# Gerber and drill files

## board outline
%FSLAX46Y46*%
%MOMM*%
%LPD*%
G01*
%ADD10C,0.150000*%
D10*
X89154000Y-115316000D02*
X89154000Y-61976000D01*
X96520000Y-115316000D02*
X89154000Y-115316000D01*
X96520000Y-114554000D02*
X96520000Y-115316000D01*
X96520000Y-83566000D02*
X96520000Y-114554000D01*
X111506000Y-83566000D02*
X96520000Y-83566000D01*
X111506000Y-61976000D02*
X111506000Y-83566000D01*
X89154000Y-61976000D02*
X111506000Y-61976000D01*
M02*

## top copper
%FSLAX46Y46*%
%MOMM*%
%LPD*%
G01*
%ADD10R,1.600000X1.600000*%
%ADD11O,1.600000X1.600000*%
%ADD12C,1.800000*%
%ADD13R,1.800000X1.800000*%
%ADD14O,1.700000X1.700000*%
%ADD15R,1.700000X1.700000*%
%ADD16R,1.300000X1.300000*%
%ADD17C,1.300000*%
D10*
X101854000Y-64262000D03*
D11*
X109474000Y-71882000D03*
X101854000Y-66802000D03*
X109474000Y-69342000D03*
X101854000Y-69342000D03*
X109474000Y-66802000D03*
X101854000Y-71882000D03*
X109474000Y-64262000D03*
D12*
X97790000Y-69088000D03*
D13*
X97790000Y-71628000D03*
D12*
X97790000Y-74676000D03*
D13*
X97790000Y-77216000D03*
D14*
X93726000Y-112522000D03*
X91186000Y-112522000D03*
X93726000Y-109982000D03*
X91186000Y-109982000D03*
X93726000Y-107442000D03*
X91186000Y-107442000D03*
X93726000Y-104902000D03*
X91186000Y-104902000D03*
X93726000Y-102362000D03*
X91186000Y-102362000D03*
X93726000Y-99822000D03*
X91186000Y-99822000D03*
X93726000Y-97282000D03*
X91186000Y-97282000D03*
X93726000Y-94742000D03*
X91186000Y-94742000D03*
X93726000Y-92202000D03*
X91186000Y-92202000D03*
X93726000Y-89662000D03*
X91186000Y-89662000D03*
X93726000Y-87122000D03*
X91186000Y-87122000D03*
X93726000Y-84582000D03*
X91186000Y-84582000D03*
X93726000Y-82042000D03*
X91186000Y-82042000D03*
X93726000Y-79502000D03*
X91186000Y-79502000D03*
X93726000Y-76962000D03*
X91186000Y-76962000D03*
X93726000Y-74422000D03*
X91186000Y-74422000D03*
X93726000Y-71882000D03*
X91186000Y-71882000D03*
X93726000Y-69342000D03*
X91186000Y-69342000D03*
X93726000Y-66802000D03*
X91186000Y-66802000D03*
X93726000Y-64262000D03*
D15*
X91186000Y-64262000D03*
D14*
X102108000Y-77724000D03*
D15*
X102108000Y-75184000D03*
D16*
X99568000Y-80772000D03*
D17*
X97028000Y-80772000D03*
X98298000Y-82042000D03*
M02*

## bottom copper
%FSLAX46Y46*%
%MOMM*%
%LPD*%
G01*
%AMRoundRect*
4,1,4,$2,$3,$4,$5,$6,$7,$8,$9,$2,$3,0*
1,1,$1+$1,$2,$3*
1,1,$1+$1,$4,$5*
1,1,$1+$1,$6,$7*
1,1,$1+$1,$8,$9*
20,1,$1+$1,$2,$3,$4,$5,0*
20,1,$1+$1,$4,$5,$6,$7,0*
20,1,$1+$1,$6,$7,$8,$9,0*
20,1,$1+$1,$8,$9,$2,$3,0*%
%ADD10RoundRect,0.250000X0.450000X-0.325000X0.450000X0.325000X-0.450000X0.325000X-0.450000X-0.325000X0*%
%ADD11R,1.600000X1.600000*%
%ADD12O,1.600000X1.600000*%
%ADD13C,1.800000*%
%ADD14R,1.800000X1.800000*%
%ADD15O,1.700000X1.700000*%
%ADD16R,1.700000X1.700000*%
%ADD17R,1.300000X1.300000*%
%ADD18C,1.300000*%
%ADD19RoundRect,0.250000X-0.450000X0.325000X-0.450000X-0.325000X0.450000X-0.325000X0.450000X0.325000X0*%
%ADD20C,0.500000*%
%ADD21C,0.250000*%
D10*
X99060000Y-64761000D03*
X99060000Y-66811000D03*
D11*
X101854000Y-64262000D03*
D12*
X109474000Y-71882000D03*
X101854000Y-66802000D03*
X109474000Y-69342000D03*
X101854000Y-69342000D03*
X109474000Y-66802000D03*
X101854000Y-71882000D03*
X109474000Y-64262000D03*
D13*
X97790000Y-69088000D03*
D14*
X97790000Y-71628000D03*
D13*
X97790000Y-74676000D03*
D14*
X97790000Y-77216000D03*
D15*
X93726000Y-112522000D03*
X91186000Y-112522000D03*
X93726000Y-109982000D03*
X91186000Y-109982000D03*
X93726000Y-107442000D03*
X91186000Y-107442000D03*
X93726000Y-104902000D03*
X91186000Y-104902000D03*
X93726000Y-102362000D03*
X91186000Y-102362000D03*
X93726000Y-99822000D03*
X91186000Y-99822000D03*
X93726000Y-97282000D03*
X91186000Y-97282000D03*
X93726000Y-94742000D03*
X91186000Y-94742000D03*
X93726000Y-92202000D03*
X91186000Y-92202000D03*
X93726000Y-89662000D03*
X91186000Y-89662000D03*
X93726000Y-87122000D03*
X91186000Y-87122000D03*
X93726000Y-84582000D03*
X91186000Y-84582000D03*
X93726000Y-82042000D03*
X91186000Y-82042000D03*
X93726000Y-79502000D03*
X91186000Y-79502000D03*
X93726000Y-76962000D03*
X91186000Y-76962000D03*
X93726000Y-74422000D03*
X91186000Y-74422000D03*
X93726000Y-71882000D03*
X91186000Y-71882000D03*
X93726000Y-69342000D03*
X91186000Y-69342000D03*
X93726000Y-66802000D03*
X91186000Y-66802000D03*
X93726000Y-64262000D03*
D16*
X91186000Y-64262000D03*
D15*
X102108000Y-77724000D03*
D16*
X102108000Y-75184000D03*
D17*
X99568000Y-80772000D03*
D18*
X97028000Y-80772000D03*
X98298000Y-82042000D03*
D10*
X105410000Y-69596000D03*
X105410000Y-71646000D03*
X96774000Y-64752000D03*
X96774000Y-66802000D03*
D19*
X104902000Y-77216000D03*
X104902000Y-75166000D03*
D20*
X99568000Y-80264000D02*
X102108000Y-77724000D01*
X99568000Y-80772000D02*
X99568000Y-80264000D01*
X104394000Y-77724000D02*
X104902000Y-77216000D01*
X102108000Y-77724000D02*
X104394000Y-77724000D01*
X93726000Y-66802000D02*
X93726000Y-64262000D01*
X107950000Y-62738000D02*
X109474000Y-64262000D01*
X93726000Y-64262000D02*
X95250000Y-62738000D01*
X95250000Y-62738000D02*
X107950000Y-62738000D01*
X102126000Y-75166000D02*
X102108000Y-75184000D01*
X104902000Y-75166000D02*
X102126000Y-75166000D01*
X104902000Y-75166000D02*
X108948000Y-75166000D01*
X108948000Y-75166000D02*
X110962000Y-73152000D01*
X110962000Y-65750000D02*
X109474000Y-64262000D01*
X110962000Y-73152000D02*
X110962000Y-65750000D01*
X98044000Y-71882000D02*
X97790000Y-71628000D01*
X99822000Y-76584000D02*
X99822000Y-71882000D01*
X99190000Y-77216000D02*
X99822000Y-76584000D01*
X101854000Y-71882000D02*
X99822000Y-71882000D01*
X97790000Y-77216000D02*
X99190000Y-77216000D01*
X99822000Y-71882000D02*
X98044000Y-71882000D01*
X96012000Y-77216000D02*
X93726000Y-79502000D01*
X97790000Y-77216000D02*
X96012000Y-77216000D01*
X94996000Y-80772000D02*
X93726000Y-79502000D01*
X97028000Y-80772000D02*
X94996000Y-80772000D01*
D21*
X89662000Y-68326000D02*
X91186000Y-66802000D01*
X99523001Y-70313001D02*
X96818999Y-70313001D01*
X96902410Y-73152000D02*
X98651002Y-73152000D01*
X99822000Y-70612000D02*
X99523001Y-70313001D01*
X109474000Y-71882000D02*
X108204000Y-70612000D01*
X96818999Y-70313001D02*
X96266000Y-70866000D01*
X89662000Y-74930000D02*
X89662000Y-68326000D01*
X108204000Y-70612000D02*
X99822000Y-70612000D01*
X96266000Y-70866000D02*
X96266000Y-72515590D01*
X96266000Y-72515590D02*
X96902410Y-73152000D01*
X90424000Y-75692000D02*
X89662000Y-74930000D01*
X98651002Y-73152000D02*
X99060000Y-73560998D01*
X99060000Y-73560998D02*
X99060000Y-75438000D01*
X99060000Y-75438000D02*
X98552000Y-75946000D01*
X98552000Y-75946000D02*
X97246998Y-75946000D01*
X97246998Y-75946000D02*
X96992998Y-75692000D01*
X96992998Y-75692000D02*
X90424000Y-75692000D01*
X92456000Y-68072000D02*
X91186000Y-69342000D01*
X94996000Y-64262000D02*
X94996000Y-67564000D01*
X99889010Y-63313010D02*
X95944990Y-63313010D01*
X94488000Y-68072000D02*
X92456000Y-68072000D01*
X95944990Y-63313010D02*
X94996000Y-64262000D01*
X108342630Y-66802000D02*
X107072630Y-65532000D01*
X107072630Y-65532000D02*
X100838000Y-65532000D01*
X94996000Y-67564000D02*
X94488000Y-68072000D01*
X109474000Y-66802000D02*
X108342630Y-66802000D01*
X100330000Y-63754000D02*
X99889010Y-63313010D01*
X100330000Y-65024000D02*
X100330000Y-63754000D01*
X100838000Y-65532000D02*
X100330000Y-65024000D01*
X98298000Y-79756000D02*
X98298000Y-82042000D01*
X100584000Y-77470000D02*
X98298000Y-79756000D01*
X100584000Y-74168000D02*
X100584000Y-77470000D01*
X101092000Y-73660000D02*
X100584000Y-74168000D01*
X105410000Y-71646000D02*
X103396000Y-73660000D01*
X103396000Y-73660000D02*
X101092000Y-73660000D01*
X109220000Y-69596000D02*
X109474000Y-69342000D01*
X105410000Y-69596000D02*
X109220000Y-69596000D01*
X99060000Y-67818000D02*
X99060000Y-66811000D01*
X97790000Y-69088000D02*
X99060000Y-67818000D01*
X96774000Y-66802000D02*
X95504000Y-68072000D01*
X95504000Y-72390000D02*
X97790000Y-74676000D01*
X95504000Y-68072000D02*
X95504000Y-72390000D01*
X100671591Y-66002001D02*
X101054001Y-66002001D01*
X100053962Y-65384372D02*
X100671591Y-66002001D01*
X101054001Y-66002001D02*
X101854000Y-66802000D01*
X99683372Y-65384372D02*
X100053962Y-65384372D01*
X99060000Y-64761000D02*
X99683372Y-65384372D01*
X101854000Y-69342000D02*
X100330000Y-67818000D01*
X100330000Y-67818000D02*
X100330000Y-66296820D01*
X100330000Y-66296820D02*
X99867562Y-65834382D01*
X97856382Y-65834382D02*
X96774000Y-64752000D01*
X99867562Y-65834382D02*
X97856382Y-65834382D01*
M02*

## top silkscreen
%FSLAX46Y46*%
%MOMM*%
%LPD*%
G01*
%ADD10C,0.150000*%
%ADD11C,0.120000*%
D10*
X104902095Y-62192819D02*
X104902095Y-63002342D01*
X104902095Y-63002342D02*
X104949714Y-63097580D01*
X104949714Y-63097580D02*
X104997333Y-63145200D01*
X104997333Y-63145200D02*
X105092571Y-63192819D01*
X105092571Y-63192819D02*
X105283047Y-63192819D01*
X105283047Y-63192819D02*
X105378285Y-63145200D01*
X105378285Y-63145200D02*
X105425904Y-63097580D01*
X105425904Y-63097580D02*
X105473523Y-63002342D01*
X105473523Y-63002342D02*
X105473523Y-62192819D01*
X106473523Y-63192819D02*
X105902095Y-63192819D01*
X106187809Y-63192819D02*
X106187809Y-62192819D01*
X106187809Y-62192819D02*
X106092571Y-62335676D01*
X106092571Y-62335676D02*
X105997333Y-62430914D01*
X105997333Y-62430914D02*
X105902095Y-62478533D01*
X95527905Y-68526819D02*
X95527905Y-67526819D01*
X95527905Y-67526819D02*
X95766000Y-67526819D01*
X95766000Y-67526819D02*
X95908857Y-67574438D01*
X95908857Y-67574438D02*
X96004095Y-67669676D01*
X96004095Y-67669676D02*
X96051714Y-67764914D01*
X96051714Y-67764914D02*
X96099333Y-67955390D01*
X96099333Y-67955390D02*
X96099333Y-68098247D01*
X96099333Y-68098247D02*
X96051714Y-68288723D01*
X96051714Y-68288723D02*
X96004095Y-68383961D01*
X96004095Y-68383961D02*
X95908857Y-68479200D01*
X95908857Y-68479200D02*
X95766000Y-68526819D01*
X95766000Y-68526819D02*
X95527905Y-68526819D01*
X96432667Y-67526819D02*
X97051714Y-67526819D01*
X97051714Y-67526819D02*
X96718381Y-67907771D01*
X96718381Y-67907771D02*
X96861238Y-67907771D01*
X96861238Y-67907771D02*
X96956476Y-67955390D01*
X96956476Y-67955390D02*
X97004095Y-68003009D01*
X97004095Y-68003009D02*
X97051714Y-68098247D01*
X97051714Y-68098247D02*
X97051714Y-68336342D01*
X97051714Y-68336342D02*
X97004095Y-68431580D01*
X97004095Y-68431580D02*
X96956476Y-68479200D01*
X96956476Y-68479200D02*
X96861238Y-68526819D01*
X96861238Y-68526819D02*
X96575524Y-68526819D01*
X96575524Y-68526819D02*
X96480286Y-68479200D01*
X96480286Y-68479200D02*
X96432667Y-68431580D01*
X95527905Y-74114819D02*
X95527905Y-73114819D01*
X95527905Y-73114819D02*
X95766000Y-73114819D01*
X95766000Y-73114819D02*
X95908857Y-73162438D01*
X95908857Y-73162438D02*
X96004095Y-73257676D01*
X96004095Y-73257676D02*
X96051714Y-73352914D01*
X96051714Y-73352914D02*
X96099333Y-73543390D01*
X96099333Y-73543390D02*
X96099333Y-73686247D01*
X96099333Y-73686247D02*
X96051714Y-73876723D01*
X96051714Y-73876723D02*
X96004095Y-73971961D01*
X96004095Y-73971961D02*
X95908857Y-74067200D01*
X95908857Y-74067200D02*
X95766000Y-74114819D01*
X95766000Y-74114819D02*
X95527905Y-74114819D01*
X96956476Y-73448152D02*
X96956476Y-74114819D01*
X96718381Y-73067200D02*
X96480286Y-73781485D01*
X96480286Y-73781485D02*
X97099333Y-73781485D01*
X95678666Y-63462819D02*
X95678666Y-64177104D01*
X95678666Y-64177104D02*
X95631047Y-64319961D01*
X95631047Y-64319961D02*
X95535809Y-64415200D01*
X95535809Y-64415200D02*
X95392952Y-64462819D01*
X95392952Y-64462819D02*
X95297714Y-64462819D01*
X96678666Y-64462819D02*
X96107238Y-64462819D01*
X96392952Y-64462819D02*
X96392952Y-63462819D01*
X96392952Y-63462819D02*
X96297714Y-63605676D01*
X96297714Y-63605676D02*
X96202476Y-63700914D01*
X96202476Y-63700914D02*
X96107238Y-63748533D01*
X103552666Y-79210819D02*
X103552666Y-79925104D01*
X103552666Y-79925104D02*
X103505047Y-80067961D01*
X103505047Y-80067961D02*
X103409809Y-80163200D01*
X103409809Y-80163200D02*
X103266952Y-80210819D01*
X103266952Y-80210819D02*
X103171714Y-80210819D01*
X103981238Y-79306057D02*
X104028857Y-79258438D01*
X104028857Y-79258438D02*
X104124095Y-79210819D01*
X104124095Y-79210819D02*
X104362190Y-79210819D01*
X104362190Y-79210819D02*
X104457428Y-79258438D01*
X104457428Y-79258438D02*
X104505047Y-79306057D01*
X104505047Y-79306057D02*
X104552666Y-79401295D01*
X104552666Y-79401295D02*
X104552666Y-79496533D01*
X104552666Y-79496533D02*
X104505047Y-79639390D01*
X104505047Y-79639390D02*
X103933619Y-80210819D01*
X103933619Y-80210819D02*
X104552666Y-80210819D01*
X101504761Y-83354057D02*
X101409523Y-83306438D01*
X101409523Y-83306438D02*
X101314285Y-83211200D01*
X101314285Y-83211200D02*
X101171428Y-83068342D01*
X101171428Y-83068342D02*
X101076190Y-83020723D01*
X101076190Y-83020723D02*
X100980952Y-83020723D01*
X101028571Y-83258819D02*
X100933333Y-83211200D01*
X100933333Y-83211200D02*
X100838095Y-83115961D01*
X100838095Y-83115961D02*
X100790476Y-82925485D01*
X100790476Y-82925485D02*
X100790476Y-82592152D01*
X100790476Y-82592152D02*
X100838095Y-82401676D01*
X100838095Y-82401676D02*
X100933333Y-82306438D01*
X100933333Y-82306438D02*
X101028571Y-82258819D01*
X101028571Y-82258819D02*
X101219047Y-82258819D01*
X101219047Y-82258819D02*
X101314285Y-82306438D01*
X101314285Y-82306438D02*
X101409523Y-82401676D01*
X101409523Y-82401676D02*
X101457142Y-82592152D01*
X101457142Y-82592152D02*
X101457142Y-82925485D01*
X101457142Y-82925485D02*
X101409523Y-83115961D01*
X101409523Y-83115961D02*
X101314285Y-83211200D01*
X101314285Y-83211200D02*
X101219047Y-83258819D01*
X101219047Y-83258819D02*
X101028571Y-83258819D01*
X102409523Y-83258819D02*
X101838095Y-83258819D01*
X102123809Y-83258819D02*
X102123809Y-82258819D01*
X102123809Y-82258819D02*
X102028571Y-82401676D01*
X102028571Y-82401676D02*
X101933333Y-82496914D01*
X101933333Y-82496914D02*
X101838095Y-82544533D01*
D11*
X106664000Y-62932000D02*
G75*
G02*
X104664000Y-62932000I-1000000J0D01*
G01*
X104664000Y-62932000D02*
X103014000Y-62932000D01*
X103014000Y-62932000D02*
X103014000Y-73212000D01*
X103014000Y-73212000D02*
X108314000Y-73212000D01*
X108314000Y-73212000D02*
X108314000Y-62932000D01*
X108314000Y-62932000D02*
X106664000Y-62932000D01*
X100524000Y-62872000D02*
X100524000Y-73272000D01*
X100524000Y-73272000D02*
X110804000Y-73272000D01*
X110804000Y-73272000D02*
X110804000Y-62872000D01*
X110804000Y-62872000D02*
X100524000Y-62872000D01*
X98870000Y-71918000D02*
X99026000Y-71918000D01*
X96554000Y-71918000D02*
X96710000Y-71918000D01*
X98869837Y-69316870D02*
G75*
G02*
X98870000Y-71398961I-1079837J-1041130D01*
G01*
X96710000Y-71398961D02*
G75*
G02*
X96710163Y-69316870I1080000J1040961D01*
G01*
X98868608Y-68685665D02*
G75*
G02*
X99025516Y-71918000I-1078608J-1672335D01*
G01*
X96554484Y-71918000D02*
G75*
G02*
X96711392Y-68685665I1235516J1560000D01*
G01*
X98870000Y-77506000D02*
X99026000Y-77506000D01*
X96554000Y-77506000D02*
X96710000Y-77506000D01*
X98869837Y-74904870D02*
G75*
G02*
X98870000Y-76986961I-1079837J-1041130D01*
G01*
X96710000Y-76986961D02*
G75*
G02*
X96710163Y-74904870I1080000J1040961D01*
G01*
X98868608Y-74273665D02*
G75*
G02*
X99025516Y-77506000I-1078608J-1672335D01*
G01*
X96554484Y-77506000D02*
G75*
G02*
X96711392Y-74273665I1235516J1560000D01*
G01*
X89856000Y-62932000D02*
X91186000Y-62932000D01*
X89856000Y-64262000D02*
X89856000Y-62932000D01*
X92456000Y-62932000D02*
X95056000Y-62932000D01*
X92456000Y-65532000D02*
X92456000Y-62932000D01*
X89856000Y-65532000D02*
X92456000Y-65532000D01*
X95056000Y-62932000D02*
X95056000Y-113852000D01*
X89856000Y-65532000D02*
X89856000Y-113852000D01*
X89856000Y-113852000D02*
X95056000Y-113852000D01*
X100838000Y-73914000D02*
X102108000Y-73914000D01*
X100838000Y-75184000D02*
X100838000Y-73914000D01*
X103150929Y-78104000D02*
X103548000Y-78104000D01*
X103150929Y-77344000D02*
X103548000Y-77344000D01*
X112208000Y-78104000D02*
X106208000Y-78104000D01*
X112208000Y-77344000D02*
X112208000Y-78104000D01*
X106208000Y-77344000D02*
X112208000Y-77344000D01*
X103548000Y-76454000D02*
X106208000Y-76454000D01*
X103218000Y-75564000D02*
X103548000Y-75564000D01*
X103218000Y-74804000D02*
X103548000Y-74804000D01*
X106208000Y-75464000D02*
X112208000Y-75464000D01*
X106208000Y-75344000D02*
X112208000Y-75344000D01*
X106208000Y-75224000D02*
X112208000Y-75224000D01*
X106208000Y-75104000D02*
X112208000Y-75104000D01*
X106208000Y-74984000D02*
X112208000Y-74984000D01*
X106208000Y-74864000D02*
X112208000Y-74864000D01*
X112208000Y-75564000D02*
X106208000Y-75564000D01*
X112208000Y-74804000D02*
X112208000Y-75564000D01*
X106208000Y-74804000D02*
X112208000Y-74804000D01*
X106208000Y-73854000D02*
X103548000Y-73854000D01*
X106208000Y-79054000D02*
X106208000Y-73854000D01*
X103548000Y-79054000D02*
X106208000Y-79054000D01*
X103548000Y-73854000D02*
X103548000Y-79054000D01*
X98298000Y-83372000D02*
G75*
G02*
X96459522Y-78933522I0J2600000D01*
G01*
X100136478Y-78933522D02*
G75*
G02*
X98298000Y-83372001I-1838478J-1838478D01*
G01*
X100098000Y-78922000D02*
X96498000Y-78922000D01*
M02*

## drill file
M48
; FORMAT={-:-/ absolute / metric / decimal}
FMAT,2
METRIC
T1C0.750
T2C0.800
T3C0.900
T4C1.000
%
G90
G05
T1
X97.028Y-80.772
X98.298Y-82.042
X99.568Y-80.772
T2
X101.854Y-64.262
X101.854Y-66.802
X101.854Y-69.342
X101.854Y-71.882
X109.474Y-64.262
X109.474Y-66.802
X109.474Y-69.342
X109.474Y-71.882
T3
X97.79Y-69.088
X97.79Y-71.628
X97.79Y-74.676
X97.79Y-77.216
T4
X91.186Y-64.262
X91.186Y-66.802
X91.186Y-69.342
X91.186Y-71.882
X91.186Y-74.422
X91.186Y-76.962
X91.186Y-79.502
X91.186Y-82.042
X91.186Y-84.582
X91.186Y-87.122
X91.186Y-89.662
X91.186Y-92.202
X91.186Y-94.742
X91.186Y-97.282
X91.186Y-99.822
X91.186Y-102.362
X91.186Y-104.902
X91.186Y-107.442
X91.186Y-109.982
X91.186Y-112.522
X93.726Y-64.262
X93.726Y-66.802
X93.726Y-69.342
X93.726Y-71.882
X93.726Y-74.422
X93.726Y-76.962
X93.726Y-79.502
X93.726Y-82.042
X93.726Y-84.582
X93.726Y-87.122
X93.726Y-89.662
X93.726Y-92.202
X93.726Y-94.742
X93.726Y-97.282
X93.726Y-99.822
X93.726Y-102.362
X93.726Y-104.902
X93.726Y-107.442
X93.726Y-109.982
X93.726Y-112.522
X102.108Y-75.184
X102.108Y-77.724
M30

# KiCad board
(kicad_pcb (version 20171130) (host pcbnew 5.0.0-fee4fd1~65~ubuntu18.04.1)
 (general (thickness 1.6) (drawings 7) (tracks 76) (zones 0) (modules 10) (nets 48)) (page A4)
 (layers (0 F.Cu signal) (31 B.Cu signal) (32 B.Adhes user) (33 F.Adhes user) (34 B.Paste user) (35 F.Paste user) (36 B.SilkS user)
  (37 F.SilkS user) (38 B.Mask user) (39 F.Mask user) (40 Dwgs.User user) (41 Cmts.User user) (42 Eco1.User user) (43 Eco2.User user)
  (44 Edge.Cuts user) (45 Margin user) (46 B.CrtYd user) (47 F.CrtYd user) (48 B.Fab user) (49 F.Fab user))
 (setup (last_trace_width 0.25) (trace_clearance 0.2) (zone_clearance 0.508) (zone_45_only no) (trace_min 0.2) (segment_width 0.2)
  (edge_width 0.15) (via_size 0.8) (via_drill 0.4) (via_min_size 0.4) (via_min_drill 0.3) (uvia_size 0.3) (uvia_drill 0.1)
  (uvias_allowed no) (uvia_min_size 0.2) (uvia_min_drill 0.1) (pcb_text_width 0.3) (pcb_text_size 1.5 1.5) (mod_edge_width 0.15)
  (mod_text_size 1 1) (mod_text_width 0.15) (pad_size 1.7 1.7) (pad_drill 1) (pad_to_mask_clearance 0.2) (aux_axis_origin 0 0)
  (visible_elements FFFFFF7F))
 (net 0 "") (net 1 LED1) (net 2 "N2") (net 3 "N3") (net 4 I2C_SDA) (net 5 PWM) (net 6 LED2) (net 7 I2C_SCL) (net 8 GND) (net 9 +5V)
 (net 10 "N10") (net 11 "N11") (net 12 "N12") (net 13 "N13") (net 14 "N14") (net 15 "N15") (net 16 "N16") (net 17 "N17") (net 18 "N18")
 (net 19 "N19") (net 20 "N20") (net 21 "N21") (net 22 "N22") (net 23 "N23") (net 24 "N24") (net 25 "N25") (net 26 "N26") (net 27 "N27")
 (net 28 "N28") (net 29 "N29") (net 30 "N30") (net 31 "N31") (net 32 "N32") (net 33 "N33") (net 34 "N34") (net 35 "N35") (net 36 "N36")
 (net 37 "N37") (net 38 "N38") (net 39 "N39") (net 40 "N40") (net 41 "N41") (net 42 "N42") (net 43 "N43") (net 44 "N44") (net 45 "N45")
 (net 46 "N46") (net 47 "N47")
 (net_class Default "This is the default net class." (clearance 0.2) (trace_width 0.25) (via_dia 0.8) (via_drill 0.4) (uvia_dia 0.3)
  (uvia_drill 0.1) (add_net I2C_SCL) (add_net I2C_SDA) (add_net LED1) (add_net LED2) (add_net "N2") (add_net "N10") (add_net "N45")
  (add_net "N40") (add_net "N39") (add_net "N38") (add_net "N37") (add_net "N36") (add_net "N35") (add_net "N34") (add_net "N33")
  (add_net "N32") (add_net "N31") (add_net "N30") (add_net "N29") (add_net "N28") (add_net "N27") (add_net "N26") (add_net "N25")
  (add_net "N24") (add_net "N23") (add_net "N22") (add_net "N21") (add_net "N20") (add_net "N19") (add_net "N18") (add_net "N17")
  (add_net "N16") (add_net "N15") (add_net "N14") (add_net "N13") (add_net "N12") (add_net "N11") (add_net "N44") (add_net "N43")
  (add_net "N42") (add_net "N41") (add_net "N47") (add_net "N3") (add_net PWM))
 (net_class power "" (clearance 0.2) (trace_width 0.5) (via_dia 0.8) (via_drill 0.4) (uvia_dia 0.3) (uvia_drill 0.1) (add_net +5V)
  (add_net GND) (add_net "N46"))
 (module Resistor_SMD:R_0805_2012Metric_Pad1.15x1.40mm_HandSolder (layer B.Cu) (at 99.06 65.786 90)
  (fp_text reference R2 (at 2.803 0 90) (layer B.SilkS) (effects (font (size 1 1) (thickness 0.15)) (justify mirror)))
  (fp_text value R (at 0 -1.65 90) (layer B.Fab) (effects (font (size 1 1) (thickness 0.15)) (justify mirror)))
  (pad 2 smd roundrect (at 1.025 0 90) (size 1.15 1.4) (layers B.Cu B.Paste B.Mask) (roundrect_rratio 0.217391) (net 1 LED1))
  (pad 1 smd roundrect (at -1.025 0 90) (size 1.15 1.4) (layers B.Cu B.Paste B.Mask) (roundrect_rratio 0.217391) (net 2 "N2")))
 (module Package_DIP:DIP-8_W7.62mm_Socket (layer F.Cu) (at 101.854 64.262)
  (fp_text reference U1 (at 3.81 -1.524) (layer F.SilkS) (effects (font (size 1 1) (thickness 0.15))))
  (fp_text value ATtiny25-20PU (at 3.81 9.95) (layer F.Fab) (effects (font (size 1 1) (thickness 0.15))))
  (fp_arc (start 3.81 -1.33) (end 2.81 -1.33) (angle -180) (layer F.SilkS) (width 0.12))
  (fp_line (start 2.81 -1.33) (end 1.16 -1.33) (layer F.SilkS) (width 0.12))
  (fp_line (start 1.16 -1.33) (end 1.16 8.95) (layer F.SilkS) (width 0.12))
  (fp_line (start 1.16 8.95) (end 6.46 8.95) (layer F.SilkS) (width 0.12))
  (fp_line (start 6.46 8.95) (end 6.46 -1.33) (layer F.SilkS) (width 0.12))
  (fp_line (start 6.46 -1.33) (end 4.81 -1.33) (layer F.SilkS) (width 0.12))
  (fp_line (start -1.33 -1.39) (end -1.33 9.01) (layer F.SilkS) (width 0.12))
  (fp_line (start -1.33 9.01) (end 8.95 9.01) (layer F.SilkS) (width 0.12))
  (fp_line (start 8.95 9.01) (end 8.95 -1.39) (layer F.SilkS) (width 0.12))
  (fp_line (start 8.95 -1.39) (end -1.33 -1.39) (layer F.SilkS) (width 0.12))
  (pad 1 thru_hole rect (at 0 0) (size 1.6 1.6) (drill 0.8) (layers *.Cu *.Mask) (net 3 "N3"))
  (pad 5 thru_hole oval (at 7.62 7.62) (size 1.6 1.6) (drill 0.8) (layers *.Cu *.Mask) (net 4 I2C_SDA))
  (pad 2 thru_hole oval (at 0 2.54) (size 1.6 1.6) (drill 0.8) (layers *.Cu *.Mask) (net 1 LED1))
  (pad 6 thru_hole oval (at 7.62 5.08) (size 1.6 1.6) (drill 0.8) (layers *.Cu *.Mask) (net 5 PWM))
  (pad 3 thru_hole oval (at 0 5.08) (size 1.6 1.6) (drill 0.8) (layers *.Cu *.Mask) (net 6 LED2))
  (pad 7 thru_hole oval (at 7.62 2.54) (size 1.6 1.6) (drill 0.8) (layers *.Cu *.Mask) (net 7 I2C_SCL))
  (pad 4 thru_hole oval (at 0 7.62) (size 1.6 1.6) (drill 0.8) (layers *.Cu *.Mask) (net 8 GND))
  (pad 8 thru_hole oval (at 7.62 0) (size 1.6 1.6) (drill 0.8) (layers *.Cu *.Mask) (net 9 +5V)))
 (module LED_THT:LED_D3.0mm (layer F.Cu) (at 97.79 71.628 90)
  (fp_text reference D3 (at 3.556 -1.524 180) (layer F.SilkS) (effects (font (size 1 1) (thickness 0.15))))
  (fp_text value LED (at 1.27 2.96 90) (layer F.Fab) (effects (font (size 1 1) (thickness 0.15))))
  (fp_line (start -0.29 1.08) (end -0.29 1.236) (layer F.SilkS) (width 0.12))
  (fp_line (start -0.29 -1.236) (end -0.29 -1.08) (layer F.SilkS) (width 0.12))
  (fp_arc (start 1.27 0) (end 0.229039 1.08) (angle -87.9) (layer F.SilkS) (width 0.12))
  (fp_arc (start 1.27 0) (end 0.229039 -1.08) (angle 87.9) (layer F.SilkS) (width 0.12))
  (fp_arc (start 1.27 0) (end -0.29 1.235516) (angle -108.8) (layer F.SilkS) (width 0.12))
  (fp_arc (start 1.27 0) (end -0.29 -1.235516) (angle 108.8) (layer F.SilkS) (width 0.12))
  (pad 2 thru_hole circle (at 2.54 0 90) (size 1.8 1.8) (drill 0.9) (layers *.Cu *.Mask) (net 2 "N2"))
  (pad 1 thru_hole rect (at 0 0 90) (size 1.8 1.8) (drill 0.9) (layers *.Cu *.Mask) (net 8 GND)))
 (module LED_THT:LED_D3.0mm (layer F.Cu) (at 97.79 77.216 90)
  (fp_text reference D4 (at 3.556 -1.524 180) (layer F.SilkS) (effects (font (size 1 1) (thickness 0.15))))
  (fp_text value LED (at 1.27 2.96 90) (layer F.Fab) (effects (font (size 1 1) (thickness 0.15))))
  (fp_line (start -0.29 1.08) (end -0.29 1.236) (layer F.SilkS) (width 0.12))
  (fp_line (start -0.29 -1.236) (end -0.29 -1.08) (layer F.SilkS) (width 0.12))
  (fp_arc (start 1.27 0) (end 0.229039 1.08) (angle -87.9) (layer F.SilkS) (width 0.12))
  (fp_arc (start 1.27 0) (end 0.229039 -1.08) (angle 87.9) (layer F.SilkS) (width 0.12))
  (fp_arc (start 1.27 0) (end -0.29 1.235516) (angle -108.8) (layer F.SilkS) (width 0.12))
  (fp_arc (start 1.27 0) (end -0.29 -1.235516) (angle 108.8) (layer F.SilkS) (width 0.12))
  (pad 2 thru_hole circle (at 2.54 0 90) (size 1.8 1.8) (drill 0.9) (layers *.Cu *.Mask) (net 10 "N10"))
  (pad 1 thru_hole rect (at 0 0 90) (size 1.8 1.8) (drill 0.9) (layers *.Cu *.Mask) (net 8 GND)))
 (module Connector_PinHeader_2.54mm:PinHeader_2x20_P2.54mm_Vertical (layer F.Cu) (at 91.186 64.262)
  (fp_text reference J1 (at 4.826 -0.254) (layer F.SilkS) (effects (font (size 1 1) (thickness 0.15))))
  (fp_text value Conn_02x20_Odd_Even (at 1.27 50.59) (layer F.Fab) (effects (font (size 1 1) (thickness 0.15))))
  (fp_line (start -1.33 -1.33) (end 0 -1.33) (layer F.SilkS) (width 0.12))
  (fp_line (start -1.33 0) (end -1.33 -1.33) (layer F.SilkS) (width 0.12))
  (fp_line (start 1.27 -1.33) (end 3.87 -1.33) (layer F.SilkS) (width 0.12))
  (fp_line (start 1.27 1.27) (end 1.27 -1.33) (layer F.SilkS) (width 0.12))
  (fp_line (start -1.33 1.27) (end 1.27 1.27) (layer F.SilkS) (width 0.12))
  (fp_line (start 3.87 -1.33) (end 3.87 49.59) (layer F.SilkS) (width 0.12))
  (fp_line (start -1.33 1.27) (end -1.33 49.59) (layer F.SilkS) (width 0.12))
  (fp_line (start -1.33 49.59) (end 3.87 49.59) (layer F.SilkS) (width 0.12))
  (pad 40 thru_hole oval (at 2.54 48.26) (size 1.7 1.7) (drill 1) (layers *.Cu *.Mask) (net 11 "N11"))
  (pad 39 thru_hole oval (at 0 48.26) (size 1.7 1.7) (drill 1) (layers *.Cu *.Mask) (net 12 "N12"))
  (pad 38 thru_hole oval (at 2.54 45.72) (size 1.7 1.7) (drill 1) (layers *.Cu *.Mask) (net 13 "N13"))
  (pad 37 thru_hole oval (at 0 45.72) (size 1.7 1.7) (drill 1) (layers *.Cu *.Mask) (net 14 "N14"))
  (pad 36 thru_hole oval (at 2.54 43.18) (size 1.7 1.7) (drill 1) (layers *.Cu *.Mask) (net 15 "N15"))
  (pad 35 thru_hole oval (at 0 43.18) (size 1.7 1.7) (drill 1) (layers *.Cu *.Mask) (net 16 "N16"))
  (pad 34 thru_hole oval (at 2.54 40.64) (size 1.7 1.7) (drill 1) (layers *.Cu *.Mask) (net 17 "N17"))
  (pad 33 thru_hole oval (at 0 40.64) (size 1.7 1.7) (drill 1) (layers *.Cu *.Mask) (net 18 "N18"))
  (pad 32 thru_hole oval (at 2.54 38.1) (size 1.7 1.7) (drill 1) (layers *.Cu *.Mask) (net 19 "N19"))
  (pad 31 thru_hole oval (at 0 38.1) (size 1.7 1.7) (drill 1) (layers *.Cu *.Mask) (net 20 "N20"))
  (pad 30 thru_hole oval (at 2.54 35.56) (size 1.7 1.7) (drill 1) (layers *.Cu *.Mask) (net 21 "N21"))
  (pad 29 thru_hole oval (at 0 35.56) (size 1.7 1.7) (drill 1) (layers *.Cu *.Mask) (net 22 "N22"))
  (pad 28 thru_hole oval (at 2.54 33.02) (size 1.7 1.7) (drill 1) (layers *.Cu *.Mask) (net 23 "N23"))
  (pad 27 thru_hole oval (at 0 33.02) (size 1.7 1.7) (drill 1) (layers *.Cu *.Mask) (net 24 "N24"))
  (pad 26 thru_hole oval (at 2.54 30.48) (size 1.7 1.7) (drill 1) (layers *.Cu *.Mask) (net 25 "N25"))
  (pad 25 thru_hole oval (at 0 30.48) (size 1.7 1.7) (drill 1) (layers *.Cu *.Mask) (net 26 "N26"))
  (pad 24 thru_hole oval (at 2.54 27.94) (size 1.7 1.7) (drill 1) (layers *.Cu *.Mask) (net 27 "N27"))
  (pad 23 thru_hole oval (at 0 27.94) (size 1.7 1.7) (drill 1) (layers *.Cu *.Mask) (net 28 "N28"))
  (pad 22 thru_hole oval (at 2.54 25.4) (size 1.7 1.7) (drill 1) (layers *.Cu *.Mask) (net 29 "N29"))
  (pad 21 thru_hole oval (at 0 25.4) (size 1.7 1.7) (drill 1) (layers *.Cu *.Mask) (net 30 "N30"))
  (pad 20 thru_hole oval (at 2.54 22.86) (size 1.7 1.7) (drill 1) (layers *.Cu *.Mask) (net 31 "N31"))
  (pad 19 thru_hole oval (at 0 22.86) (size 1.7 1.7) (drill 1) (layers *.Cu *.Mask) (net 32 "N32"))
  (pad 18 thru_hole oval (at 2.54 20.32) (size 1.7 1.7) (drill 1) (layers *.Cu *.Mask) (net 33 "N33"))
  (pad 17 thru_hole oval (at 0 20.32) (size 1.7 1.7) (drill 1) (layers *.Cu *.Mask) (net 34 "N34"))
  (pad 16 thru_hole oval (at 2.54 17.78) (size 1.7 1.7) (drill 1) (layers *.Cu *.Mask) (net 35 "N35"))
  (pad 15 thru_hole oval (at 0 17.78) (size 1.7 1.7) (drill 1) (layers *.Cu *.Mask) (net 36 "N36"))
  (pad 14 thru_hole oval (at 2.54 15.24) (size 1.7 1.7) (drill 1) (layers *.Cu *.Mask) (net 8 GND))
  (pad 13 thru_hole oval (at 0 15.24) (size 1.7 1.7) (drill 1) (layers *.Cu *.Mask) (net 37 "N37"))
  (pad 12 thru_hole oval (at 2.54 12.7) (size 1.7 1.7) (drill 1) (layers *.Cu *.Mask) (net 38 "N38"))
  (pad 11 thru_hole oval (at 0 12.7) (size 1.7 1.7) (drill 1) (layers *.Cu *.Mask) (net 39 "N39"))
  (pad 10 thru_hole oval (at 2.54 10.16) (size 1.7 1.7) (drill 1) (layers *.Cu *.Mask) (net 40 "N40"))
  (pad 9 thru_hole oval (at 0 10.16) (size 1.7 1.7) (drill 1) (layers *.Cu *.Mask) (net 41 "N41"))
  (pad 8 thru_hole oval (at 2.54 7.62) (size 1.7 1.7) (drill 1) (layers *.Cu *.Mask) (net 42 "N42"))
  (pad 7 thru_hole oval (at 0 7.62) (size 1.7 1.7) (drill 1) (layers *.Cu *.Mask) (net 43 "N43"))
  (pad 6 thru_hole oval (at 2.54 5.08) (size 1.7 1.7) (drill 1) (layers *.Cu *.Mask) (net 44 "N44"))
  (pad 5 thru_hole oval (at 0 5.08) (size 1.7 1.7) (drill 1) (layers *.Cu *.Mask) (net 7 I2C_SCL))
  (pad 4 thru_hole oval (at 2.54 2.54) (size 1.7 1.7) (drill 1) (layers *.Cu *.Mask) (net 9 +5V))
  (pad 3 thru_hole oval (at 0 2.54) (size 1.7 1.7) (drill 1) (layers *.Cu *.Mask) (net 4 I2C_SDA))
  (pad 2 thru_hole oval (at 2.54 0) (size 1.7 1.7) (drill 1) (layers *.Cu *.Mask) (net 9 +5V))
  (pad 1 thru_hole rect (at 0 0) (size 1.7 1.7) (drill 1) (layers *.Cu *.Mask) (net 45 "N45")))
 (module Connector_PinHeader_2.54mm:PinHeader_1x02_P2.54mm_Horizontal (layer F.Cu) (at 102.108 75.184)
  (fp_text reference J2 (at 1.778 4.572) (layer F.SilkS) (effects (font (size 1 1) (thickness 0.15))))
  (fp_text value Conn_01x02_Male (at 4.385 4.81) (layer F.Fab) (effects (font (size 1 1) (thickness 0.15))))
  (fp_line (start -1.27 -1.27) (end 0 -1.27) (layer F.SilkS) (width 0.12))
  (fp_line (start -1.27 0) (end -1.27 -1.27) (layer F.SilkS) (width 0.12))
  (fp_line (start 1.042929 2.92) (end 1.44 2.92) (layer F.SilkS) (width 0.12))
  (fp_line (start 1.042929 2.16) (end 1.44 2.16) (layer F.SilkS) (width 0.12))
  (fp_line (start 10.1 2.92) (end 4.1 2.92) (layer F.SilkS) (width 0.12))
  (fp_line (start 10.1 2.16) (end 10.1 2.92) (layer F.SilkS) (width 0.12))
  (fp_line (start 4.1 2.16) (end 10.1 2.16) (layer F.SilkS) (width 0.12))
  (fp_line (start 1.44 1.27) (end 4.1 1.27) (layer F.SilkS) (width 0.12))
  (fp_line (start 1.11 0.38) (end 1.44 0.38) (layer F.SilkS) (width 0.12))
  (fp_line (start 1.11 -0.38) (end 1.44 -0.38) (layer F.SilkS) (width 0.12))
  (fp_line (start 4.1 0.28) (end 10.1 0.28) (layer F.SilkS) (width 0.12))
  (fp_line (start 4.1 0.16) (end 10.1 0.16) (layer F.SilkS) (width 0.12))
  (fp_line (start 4.1 0.04) (end 10.1 0.04) (layer F.SilkS) (width 0.12))
  (fp_line (start 4.1 -0.08) (end 10.1 -0.08) (layer F.SilkS) (width 0.12))
  (fp_line (start 4.1 -0.2) (end 10.1 -0.2) (layer F.SilkS) (width 0.12))
  (fp_line (start 4.1 -0.32) (end 10.1 -0.32) (layer F.SilkS) (width 0.12))
  (fp_line (start 10.1 0.38) (end 4.1 0.38) (layer F.SilkS) (width 0.12))
  (fp_line (start 10.1 -0.38) (end 10.1 0.38) (layer F.SilkS) (width 0.12))
  (fp_line (start 4.1 -0.38) (end 10.1 -0.38) (layer F.SilkS) (width 0.12))
  (fp_line (start 4.1 -1.33) (end 1.44 -1.33) (layer F.SilkS) (width 0.12))
  (fp_line (start 4.1 3.87) (end 4.1 -1.33) (layer F.SilkS) (width 0.12))
  (fp_line (start 1.44 3.87) (end 4.1 3.87) (layer F.SilkS) (width 0.12))
  (fp_line (start 1.44 -1.33) (end 1.44 3.87) (layer F.SilkS) (width 0.12))
  (pad 2 thru_hole oval (at 0 2.54) (size 1.7 1.7) (drill 1) (layers *.Cu *.Mask) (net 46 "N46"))
  (pad 1 thru_hole rect (at 0 0) (size 1.7 1.7) (drill 1) (layers *.Cu *.Mask) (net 9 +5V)))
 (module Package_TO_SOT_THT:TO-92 (layer F.Cu) (at 99.568 80.772 180)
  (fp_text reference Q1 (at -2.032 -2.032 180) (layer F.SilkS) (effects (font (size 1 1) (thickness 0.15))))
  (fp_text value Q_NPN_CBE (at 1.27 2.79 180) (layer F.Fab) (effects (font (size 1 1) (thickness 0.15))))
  (fp_arc (start 1.27 0) (end 1.27 -2.6) (angle 135) (layer F.SilkS) (width 0.12))
  (fp_arc (start 1.27 0) (end 1.27 -2.6) (angle -135) (layer F.SilkS) (width 0.12))
  (fp_line (start -0.53 1.85) (end 3.07 1.85) (layer F.SilkS) (width 0.12))
  (pad 1 thru_hole rect (at 0 0 270) (size 1.3 1.3) (drill 0.75) (layers *.Cu *.Mask) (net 46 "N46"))
  (pad 3 thru_hole circle (at 2.54 0 270) (size 1.3 1.3) (drill 0.75) (layers *.Cu *.Mask) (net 8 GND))
  (pad 2 thru_hole circle (at 1.27 -1.27 270) (size 1.3 1.3) (drill 0.75) (layers *.Cu *.Mask) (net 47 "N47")))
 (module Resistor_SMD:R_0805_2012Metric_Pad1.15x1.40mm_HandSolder (layer B.Cu) (at 105.41 70.621 90)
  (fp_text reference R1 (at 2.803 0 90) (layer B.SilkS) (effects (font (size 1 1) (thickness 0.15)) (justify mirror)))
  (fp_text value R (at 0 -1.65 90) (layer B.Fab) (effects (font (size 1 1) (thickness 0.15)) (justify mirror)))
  (pad 2 smd roundrect (at 1.025 0 90) (size 1.15 1.4) (layers B.Cu B.Paste B.Mask) (roundrect_rratio 0.217391) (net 5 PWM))
  (pad 1 smd roundrect (at -1.025 0 90) (size 1.15 1.4) (layers B.Cu B.Paste B.Mask) (roundrect_rratio 0.217391) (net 47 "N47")))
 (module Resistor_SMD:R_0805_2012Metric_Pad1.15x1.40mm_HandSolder (layer B.Cu) (at 96.774 65.777 90)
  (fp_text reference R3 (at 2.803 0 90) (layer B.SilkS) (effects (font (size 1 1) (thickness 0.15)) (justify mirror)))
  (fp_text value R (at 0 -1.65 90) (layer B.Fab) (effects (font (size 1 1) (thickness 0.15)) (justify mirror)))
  (pad 2 smd roundrect (at 1.025 0 90) (size 1.15 1.4) (layers B.Cu B.Paste B.Mask) (roundrect_rratio 0.217391) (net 6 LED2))
  (pad 1 smd roundrect (at -1.025 0 90) (size 1.15 1.4) (layers B.Cu B.Paste B.Mask) (roundrect_rratio 0.217391) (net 10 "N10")))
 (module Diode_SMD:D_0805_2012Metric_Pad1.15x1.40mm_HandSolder (layer B.Cu) (at 104.902 76.191 270)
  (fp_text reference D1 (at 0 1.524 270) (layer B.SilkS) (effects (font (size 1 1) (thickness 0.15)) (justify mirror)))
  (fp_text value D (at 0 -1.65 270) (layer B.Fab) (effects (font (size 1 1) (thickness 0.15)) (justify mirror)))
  (pad 2 smd roundrect (at 1.025 0 270) (size 1.15 1.4) (layers B.Cu B.Paste B.Mask) (roundrect_rratio 0.217391) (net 46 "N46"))
  (pad 1 smd roundrect (at -1.025 0 270) (size 1.15 1.4) (layers B.Cu B.Paste B.Mask) (roundrect_rratio 0.217391) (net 9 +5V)))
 (gr_line (start 89.154 115.316) (end 89.154 61.976) (layer Edge.Cuts) (width 0.15))
 (gr_line (start 96.52 115.316) (end 89.154 115.316) (layer Edge.Cuts) (width 0.15))
 (gr_line (start 96.52 114.554) (end 96.52 115.316) (layer Edge.Cuts) (width 0.15))
 (gr_line (start 96.52 83.566) (end 96.52 114.554) (layer Edge.Cuts) (width 0.15))
 (gr_line (start 111.506 83.566) (end 96.52 83.566) (layer Edge.Cuts) (width 0.15))
 (gr_line (start 111.506 61.976) (end 111.506 83.566) (layer Edge.Cuts) (width 0.15))
 (gr_line (start 89.154 61.976) (end 111.506 61.976) (layer Edge.Cuts) (width 0.15))
 (segment (start 99.568 80.264) (end 102.108 77.724) (width 0.5) (layer B.Cu) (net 46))
 (segment (start 99.568 80.772) (end 99.568 80.264) (width 0.5) (layer B.Cu) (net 46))
 (segment (start 104.394 77.724) (end 104.902 77.216) (width 0.5) (layer B.Cu) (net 46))
 (segment (start 102.108 77.724) (end 104.394 77.724) (width 0.5) (layer B.Cu) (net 46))
 (segment (start 93.726 66.802) (end 93.726 64.262) (width 0.5) (layer B.Cu) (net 9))
 (segment (start 107.95 62.738) (end 109.474 64.262) (width 0.5) (layer B.Cu) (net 9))
 (segment (start 93.726 64.262) (end 95.25 62.738) (width 0.5) (layer B.Cu) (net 9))
 (segment (start 95.25 62.738) (end 107.95 62.738) (width 0.5) (layer B.Cu) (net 9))
 (segment (start 102.126 75.166) (end 102.108 75.184) (width 0.5) (layer B.Cu) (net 9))
 (segment (start 104.902 75.166) (end 102.126 75.166) (width 0.5) (layer B.Cu) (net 9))
 (segment (start 104.902 75.166) (end 108.948 75.166) (width 0.5) (layer B.Cu) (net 9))
 (segment (start 108.948 75.166) (end 110.962 73.152) (width 0.5) (layer B.Cu) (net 9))
 (segment (start 110.962 65.75) (end 109.474 64.262) (width 0.5) (layer B.Cu) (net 9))
 (segment (start 110.962 73.152) (end 110.962 65.75) (width 0.5) (layer B.Cu) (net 9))
 (segment (start 98.044 71.882) (end 97.79 71.628) (width 0.5) (layer B.Cu) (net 8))
 (segment (start 99.822 76.584) (end 99.822 71.882) (width 0.5) (layer B.Cu) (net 8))
 (segment (start 99.19 77.216) (end 99.822 76.584) (width 0.5) (layer B.Cu) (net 8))
 (segment (start 101.854 71.882) (end 99.822 71.882) (width 0.5) (layer B.Cu) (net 8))
 (segment (start 97.79 77.216) (end 99.19 77.216) (width 0.5) (layer B.Cu) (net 8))
 (segment (start 99.822 71.882) (end 98.044 71.882) (width 0.5) (layer B.Cu) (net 8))
 (segment (start 96.012 77.216) (end 93.726 79.502) (width 0.5) (layer B.Cu) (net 8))
 (segment (start 97.79 77.216) (end 96.012 77.216) (width 0.5) (layer B.Cu) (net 8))
 (segment (start 94.996 80.772) (end 93.726 79.502) (width 0.5) (layer B.Cu) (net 8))
 (segment (start 97.028 80.772) (end 94.996 80.772) (width 0.5) (layer B.Cu) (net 8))
 (segment (start 89.662 68.326) (end 91.186 66.802) (width 0.25) (layer B.Cu) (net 4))
 (segment (start 99.523001 70.313001) (end 96.818999 70.313001) (width 0.25) (layer B.Cu) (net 4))
 (segment (start 96.90241 73.152) (end 98.651002 73.152) (width 0.25) (layer B.Cu) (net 4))
 (segment (start 99.822 70.612) (end 99.523001 70.313001) (width 0.25) (layer B.Cu) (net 4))
 (segment (start 109.474 71.882) (end 108.204 70.612) (width 0.25) (layer B.Cu) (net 4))
 (segment (start 96.818999 70.313001) (end 96.266 70.866) (width 0.25) (layer B.Cu) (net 4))
 (segment (start 89.662 74.93) (end 89.662 68.326) (width 0.25) (layer B.Cu) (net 4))
 (segment (start 108.204 70.612) (end 99.822 70.612) (width 0.25) (layer B.Cu) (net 4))
 (segment (start 96.266 70.866) (end 96.266 72.51559) (width 0.25) (layer B.Cu) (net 4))
 (segment (start 96.266 72.51559) (end 96.90241 73.152) (width 0.25) (layer B.Cu) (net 4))
 (segment (start 90.424 75.692) (end 89.662 74.93) (width 0.25) (layer B.Cu) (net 4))
 (segment (start 98.651002 73.152) (end 99.06 73.560998) (width 0.25) (layer B.Cu) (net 4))
 (segment (start 99.06 73.560998) (end 99.06 75.438) (width 0.25) (layer B.Cu) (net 4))
 (segment (start 99.06 75.438) (end 98.552 75.946) (width 0.25) (layer B.Cu) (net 4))
 (segment (start 98.552 75.946) (end 97.246998 75.946) (width 0.25) (layer B.Cu) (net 4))
 (segment (start 97.246998 75.946) (end 96.992998 75.692) (width 0.25) (layer B.Cu) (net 4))
 (segment (start 96.992998 75.692) (end 90.424 75.692) (width 0.25) (layer B.Cu) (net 4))
 (segment (start 92.456 68.072) (end 91.186 69.342) (width 0.25) (layer B.Cu) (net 7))
 (segment (start 94.996 64.262) (end 94.996 67.564) (width 0.25) (layer B.Cu) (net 7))
 (segment (start 99.88901 63.31301) (end 95.94499 63.31301) (width 0.25) (layer B.Cu) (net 7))
 (segment (start 94.488 68.072) (end 92.456 68.072) (width 0.25) (layer B.Cu) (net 7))
 (segment (start 95.94499 63.31301) (end 94.996 64.262) (width 0.25) (layer B.Cu) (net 7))
 (segment (start 108.34263 66.802) (end 107.07263 65.532) (width 0.25) (layer B.Cu) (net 7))
 (segment (start 107.07263 65.532) (end 100.838 65.532) (width 0.25) (layer B.Cu) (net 7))
 (segment (start 94.996 67.564) (end 94.488 68.072) (width 0.25) (layer B.Cu) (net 7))
 (segment (start 109.474 66.802) (end 108.34263 66.802) (width 0.25) (layer B.Cu) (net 7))
 (segment (start 100.33 63.754) (end 99.88901 63.31301) (width 0.25) (layer B.Cu) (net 7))
 (segment (start 100.33 65.024) (end 100.33 63.754) (width 0.25) (layer B.Cu) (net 7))
 (segment (start 100.838 65.532) (end 100.33 65.024) (width 0.25) (layer B.Cu) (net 7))
 (segment (start 98.298 79.756) (end 98.298 82.042) (width 0.25) (layer B.Cu) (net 47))
 (segment (start 100.584 77.47) (end 98.298 79.756) (width 0.25) (layer B.Cu) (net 47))
 (segment (start 100.584 74.168) (end 100.584 77.47) (width 0.25) (layer B.Cu) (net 47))
 (segment (start 101.092 73.66) (end 100.584 74.168) (width 0.25) (layer B.Cu) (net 47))
 (segment (start 105.41 71.646) (end 103.396 73.66) (width 0.25) (layer B.Cu) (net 47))
 (segment (start 103.396 73.66) (end 101.092 73.66) (width 0.25) (layer B.Cu) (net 47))
 (segment (start 109.22 69.596) (end 109.474 69.342) (width 0.25) (layer B.Cu) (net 5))
 (segment (start 105.41 69.596) (end 109.22 69.596) (width 0.25) (layer B.Cu) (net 5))
 (segment (start 99.06 67.818) (end 99.06 66.811) (width 0.25) (layer B.Cu) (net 2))
 (segment (start 97.79 69.088) (end 99.06 67.818) (width 0.25) (layer B.Cu) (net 2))
 (segment (start 96.774 66.802) (end 95.504 68.072) (width 0.25) (layer B.Cu) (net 10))
 (segment (start 95.504 72.39) (end 97.79 74.676) (width 0.25) (layer B.Cu) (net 10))
 (segment (start 95.504 68.072) (end 95.504 72.39) (width 0.25) (layer B.Cu) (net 10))
 (segment (start 100.671591 66.002001) (end 101.054001 66.002001) (width 0.25) (layer B.Cu) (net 1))
 (segment (start 100.053962 65.384372) (end 100.671591 66.002001) (width 0.25) (layer B.Cu) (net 1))
 (segment (start 101.054001 66.002001) (end 101.854 66.802) (width 0.25) (layer B.Cu) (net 1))
 (segment (start 99.683372 65.384372) (end 100.053962 65.384372) (width 0.25) (layer B.Cu) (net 1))
 (segment (start 99.06 64.761) (end 99.683372 65.384372) (width 0.25) (layer B.Cu) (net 1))
 (segment (start 101.854 69.342) (end 100.33 67.818) (width 0.25) (layer B.Cu) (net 6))
 (segment (start 100.33 67.818) (end 100.33 66.29682) (width 0.25) (layer B.Cu) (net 6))
 (segment (start 100.33 66.29682) (end 99.867562 65.834382) (width 0.25) (layer B.Cu) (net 6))
 (segment (start 97.856382 65.834382) (end 96.774 64.752) (width 0.25) (layer B.Cu) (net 6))
 (segment (start 99.867562 65.834382) (end 97.856382 65.834382) (width 0.25) (layer B.Cu) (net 6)))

